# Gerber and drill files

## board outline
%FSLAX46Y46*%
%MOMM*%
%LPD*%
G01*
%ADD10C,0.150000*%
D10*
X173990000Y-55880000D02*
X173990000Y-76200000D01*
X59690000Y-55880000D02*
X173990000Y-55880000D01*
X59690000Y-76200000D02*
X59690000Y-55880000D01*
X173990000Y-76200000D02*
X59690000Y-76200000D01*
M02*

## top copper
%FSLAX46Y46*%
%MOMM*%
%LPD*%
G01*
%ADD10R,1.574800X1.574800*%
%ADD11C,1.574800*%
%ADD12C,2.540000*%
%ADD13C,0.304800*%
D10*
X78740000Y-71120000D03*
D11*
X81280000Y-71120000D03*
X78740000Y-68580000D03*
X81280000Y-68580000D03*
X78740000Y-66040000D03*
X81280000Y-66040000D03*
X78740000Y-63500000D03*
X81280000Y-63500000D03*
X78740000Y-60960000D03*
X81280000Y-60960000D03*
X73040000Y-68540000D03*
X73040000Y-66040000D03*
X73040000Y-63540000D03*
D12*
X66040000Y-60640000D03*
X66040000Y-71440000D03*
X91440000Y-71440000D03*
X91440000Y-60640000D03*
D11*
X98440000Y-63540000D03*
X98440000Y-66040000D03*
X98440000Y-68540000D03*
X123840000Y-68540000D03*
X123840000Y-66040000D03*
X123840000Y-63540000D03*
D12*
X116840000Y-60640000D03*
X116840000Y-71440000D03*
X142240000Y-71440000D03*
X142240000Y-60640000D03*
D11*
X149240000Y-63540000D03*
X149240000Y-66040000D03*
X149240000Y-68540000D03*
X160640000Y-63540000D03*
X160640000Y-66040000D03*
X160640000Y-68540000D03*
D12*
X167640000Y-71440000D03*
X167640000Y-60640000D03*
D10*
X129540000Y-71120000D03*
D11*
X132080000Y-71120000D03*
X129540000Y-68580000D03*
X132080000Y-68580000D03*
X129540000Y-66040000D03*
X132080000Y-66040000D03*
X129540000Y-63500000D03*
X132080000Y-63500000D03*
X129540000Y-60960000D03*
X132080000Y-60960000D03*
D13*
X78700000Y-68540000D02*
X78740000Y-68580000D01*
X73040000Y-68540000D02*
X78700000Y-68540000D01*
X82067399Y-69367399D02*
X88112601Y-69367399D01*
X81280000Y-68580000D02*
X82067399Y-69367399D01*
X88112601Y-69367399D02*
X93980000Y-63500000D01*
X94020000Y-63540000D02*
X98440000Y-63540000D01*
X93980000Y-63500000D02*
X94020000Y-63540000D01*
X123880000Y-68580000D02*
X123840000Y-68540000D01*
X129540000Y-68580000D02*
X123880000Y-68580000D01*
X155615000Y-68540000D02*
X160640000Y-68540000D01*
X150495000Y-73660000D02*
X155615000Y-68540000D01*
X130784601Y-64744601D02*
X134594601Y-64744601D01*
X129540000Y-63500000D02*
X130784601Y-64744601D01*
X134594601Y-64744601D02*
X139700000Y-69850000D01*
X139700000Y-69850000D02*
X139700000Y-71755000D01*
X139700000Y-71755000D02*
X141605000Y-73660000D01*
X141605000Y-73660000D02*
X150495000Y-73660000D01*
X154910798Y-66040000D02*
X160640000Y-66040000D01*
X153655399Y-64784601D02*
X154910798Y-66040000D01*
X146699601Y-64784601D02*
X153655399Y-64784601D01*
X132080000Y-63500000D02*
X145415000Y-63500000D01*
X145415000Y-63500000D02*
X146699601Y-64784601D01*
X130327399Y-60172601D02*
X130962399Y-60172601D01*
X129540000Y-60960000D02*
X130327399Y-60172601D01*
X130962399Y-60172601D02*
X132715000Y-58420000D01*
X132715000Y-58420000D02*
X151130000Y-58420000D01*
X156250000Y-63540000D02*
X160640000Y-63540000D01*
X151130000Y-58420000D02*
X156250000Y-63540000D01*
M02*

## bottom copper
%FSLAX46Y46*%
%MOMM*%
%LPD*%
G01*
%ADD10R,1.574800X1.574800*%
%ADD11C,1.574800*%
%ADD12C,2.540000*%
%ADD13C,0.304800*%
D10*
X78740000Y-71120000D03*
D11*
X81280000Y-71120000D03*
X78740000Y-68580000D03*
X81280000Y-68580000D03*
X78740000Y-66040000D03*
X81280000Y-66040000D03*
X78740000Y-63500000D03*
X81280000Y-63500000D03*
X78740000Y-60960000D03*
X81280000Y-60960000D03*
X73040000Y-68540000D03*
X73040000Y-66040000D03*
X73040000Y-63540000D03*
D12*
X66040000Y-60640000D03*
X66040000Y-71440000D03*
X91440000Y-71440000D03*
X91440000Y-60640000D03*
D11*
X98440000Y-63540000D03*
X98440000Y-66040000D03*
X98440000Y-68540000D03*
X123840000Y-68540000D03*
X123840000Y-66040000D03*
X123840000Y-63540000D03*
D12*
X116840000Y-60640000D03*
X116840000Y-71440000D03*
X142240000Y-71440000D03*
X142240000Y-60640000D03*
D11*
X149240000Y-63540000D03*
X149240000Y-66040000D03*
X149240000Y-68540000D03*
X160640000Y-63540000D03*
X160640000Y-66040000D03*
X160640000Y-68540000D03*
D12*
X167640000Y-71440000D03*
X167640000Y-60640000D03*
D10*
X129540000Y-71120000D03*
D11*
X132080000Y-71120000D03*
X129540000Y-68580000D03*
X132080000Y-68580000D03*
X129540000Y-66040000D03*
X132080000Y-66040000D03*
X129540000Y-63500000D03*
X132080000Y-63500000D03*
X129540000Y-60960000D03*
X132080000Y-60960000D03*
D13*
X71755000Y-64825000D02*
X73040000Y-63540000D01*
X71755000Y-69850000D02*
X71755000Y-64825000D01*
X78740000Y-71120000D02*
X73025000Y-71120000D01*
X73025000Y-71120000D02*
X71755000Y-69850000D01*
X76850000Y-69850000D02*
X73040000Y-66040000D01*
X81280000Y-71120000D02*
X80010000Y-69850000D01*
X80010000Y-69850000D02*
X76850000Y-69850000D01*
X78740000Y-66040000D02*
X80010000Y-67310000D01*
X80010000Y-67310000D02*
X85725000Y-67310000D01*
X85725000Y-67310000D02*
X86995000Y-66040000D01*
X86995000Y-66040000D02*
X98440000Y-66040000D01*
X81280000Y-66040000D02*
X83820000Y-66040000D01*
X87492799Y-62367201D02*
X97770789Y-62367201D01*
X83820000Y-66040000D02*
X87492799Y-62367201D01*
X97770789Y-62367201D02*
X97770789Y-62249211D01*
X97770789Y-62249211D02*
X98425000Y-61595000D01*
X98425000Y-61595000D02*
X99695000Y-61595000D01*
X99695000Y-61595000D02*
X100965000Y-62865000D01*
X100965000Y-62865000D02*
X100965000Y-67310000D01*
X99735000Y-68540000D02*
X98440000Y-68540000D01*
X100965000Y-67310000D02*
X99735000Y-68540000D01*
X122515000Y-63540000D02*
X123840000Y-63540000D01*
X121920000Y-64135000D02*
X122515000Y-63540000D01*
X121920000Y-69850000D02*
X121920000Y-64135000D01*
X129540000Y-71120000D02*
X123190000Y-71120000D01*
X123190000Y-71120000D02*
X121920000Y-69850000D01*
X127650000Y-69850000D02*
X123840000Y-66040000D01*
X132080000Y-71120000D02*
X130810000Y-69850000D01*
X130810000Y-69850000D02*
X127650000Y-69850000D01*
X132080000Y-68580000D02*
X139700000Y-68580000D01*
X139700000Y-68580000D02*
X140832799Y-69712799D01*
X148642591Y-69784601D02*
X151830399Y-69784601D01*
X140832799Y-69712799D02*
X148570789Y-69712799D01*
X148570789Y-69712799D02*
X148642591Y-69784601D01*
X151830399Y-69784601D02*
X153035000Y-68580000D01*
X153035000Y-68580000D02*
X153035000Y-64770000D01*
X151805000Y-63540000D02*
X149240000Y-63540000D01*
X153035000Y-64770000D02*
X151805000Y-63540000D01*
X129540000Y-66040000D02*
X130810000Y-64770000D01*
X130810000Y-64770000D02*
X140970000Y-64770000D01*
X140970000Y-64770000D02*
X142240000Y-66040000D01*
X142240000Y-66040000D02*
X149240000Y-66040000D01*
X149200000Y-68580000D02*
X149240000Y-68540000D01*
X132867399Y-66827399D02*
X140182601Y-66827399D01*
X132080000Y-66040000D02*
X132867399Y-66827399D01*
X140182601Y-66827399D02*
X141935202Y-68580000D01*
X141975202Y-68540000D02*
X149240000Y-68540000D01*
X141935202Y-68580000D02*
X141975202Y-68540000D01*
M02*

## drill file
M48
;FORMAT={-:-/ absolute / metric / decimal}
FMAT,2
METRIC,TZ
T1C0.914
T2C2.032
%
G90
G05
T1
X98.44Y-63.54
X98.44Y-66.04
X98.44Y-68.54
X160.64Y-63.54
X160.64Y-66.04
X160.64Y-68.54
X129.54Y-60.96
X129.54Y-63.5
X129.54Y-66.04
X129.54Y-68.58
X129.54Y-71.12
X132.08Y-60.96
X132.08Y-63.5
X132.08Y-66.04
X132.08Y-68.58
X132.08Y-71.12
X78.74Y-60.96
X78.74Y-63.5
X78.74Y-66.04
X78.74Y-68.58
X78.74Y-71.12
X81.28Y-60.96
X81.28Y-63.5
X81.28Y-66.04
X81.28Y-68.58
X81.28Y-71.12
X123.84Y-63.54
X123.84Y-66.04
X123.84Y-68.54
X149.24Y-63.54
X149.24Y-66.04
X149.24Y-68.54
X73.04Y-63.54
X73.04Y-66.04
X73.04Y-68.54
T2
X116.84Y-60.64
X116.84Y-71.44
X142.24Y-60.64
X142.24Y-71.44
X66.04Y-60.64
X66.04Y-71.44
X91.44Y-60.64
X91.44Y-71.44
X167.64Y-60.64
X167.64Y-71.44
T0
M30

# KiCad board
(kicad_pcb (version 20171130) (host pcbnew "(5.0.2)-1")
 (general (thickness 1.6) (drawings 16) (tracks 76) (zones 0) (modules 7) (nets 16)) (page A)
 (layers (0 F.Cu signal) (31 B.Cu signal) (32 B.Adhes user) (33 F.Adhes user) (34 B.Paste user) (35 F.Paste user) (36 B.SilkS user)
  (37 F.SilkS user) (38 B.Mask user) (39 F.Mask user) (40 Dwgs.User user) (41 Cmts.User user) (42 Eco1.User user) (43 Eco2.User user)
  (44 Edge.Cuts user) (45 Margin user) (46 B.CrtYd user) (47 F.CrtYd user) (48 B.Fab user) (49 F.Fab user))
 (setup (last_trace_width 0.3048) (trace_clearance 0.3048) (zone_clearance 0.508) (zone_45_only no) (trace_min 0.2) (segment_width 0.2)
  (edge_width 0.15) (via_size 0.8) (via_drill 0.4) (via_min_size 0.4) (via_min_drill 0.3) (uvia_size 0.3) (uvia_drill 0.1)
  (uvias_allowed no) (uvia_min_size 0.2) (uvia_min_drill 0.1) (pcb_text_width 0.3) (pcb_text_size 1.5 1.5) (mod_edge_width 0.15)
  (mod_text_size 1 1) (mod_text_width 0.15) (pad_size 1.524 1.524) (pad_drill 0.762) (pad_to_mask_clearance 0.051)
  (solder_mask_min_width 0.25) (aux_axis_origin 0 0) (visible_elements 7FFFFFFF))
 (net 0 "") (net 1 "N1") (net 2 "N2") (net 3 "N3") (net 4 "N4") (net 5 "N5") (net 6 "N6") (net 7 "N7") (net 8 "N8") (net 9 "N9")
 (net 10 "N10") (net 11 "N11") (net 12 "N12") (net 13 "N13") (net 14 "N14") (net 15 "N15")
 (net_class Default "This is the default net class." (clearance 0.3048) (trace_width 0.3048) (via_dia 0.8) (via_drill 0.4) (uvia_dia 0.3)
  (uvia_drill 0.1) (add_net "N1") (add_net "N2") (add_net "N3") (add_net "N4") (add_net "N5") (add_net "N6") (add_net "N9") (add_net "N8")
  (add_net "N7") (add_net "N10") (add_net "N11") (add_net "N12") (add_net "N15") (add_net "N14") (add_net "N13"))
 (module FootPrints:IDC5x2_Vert (layer B.Cu) (at 80.01 66.04 270)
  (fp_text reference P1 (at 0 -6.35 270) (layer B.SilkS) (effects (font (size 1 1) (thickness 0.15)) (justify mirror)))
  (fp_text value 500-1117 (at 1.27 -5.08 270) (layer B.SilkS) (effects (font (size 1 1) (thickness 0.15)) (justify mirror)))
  (pad 1 thru_hole rect (at 5.08 1.27 270) (size 1.5748 1.5748) (drill 0.9144) (layers *.Cu *.Mask B.SilkS) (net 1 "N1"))
  (pad 2 thru_hole circle (at 5.08 -1.27 270) (size 1.5748 1.5748) (drill 0.9144) (layers *.Cu *.Mask B.SilkS) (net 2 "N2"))
  (pad 3 thru_hole circle (at 2.54 1.27 270) (size 1.5748 1.5748) (drill 0.9144) (layers *.Cu *.Mask B.SilkS) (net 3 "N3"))
  (pad 4 thru_hole circle (at 2.54 -1.27 270) (size 1.5748 1.5748) (drill 0.9144) (layers *.Cu *.Mask B.SilkS) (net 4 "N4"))
  (pad 5 thru_hole circle (at 0 1.27 270) (size 1.5748 1.5748) (drill 0.9144) (layers *.Cu *.Mask B.SilkS) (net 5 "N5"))
  (pad 6 thru_hole circle (at 0 -1.27 270) (size 1.5748 1.5748) (drill 0.9144) (layers *.Cu *.Mask B.SilkS) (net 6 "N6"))
  (pad 7 thru_hole circle (at -2.54 1.27 270) (size 1.5748 1.5748) (drill 0.9144) (layers *.Cu *.Mask B.SilkS))
  (pad 8 thru_hole circle (at -2.54 -1.27 270) (size 1.5748 1.5748) (drill 0.9144) (layers *.Cu *.Mask B.SilkS))
  (pad 9 thru_hole circle (at -5.08 1.27 270) (size 1.5748 1.5748) (drill 0.9144) (layers *.Cu *.Mask B.SilkS))
  (pad 10 thru_hole circle (at -5.08 -1.27 270) (size 1.5748 1.5748) (drill 0.9144) (layers *.Cu *.Mask B.SilkS)))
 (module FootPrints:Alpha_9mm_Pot (layer F.Cu) (at 66.04 66.04 90)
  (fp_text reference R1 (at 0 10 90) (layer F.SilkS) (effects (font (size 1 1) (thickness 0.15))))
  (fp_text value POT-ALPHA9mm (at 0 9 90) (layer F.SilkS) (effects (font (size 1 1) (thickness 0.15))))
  (pad 1 thru_hole circle (at -2.5 7 90) (size 1.5748 1.5748) (drill 0.9144) (layers *.Cu *.Mask) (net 3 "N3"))
  (pad 2 thru_hole circle (at 0 7 90) (size 1.5748 1.5748) (drill 0.9144) (layers *.Cu *.Mask) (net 2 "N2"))
  (pad 3 thru_hole circle (at 2.5 7 90) (size 1.5748 1.5748) (drill 0.9144) (layers *.Cu *.Mask) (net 1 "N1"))
  (pad 4 thru_hole circle (at 5.4 0 90) (size 2.54 2.54) (drill 2.032) (layers *.Cu *.Mask))
  (pad 5 thru_hole circle (at -5.4 0 90) (size 2.54 2.54) (drill 2.032) (layers *.Cu *.Mask)))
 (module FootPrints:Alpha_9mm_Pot (layer F.Cu) (at 91.44 66.04 90)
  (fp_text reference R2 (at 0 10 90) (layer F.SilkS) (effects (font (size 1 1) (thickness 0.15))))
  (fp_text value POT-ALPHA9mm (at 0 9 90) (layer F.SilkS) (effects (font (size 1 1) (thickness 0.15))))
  (pad 5 thru_hole circle (at -5.4 0 90) (size 2.54 2.54) (drill 2.032) (layers *.Cu *.Mask))
  (pad 4 thru_hole circle (at 5.4 0 90) (size 2.54 2.54) (drill 2.032) (layers *.Cu *.Mask))
  (pad 3 thru_hole circle (at 2.5 7 90) (size 1.5748 1.5748) (drill 0.9144) (layers *.Cu *.Mask) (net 4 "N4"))
  (pad 2 thru_hole circle (at 0 7 90) (size 1.5748 1.5748) (drill 0.9144) (layers *.Cu *.Mask) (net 5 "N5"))
  (pad 1 thru_hole circle (at -2.5 7 90) (size 1.5748 1.5748) (drill 0.9144) (layers *.Cu *.Mask) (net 6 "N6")))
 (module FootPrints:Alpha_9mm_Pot (layer F.Cu) (at 116.84 66.04 90)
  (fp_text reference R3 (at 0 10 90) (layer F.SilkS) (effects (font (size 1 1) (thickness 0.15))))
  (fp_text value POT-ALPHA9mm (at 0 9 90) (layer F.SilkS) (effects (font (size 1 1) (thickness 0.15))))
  (pad 1 thru_hole circle (at -2.5 7 90) (size 1.5748 1.5748) (drill 0.9144) (layers *.Cu *.Mask) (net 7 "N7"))
  (pad 2 thru_hole circle (at 0 7 90) (size 1.5748 1.5748) (drill 0.9144) (layers *.Cu *.Mask) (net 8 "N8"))
  (pad 3 thru_hole circle (at 2.5 7 90) (size 1.5748 1.5748) (drill 0.9144) (layers *.Cu *.Mask) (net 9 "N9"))
  (pad 4 thru_hole circle (at 5.4 0 90) (size 2.54 2.54) (drill 2.032) (layers *.Cu *.Mask))
  (pad 5 thru_hole circle (at -5.4 0 90) (size 2.54 2.54) (drill 2.032) (layers *.Cu *.Mask)))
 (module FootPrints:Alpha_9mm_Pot (layer F.Cu) (at 142.24 66.04 90)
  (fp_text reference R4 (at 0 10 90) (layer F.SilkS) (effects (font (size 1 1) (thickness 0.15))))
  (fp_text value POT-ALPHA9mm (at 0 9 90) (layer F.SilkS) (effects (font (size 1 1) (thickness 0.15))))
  (pad 5 thru_hole circle (at -5.4 0 90) (size 2.54 2.54) (drill 2.032) (layers *.Cu *.Mask))
  (pad 4 thru_hole circle (at 5.4 0 90) (size 2.54 2.54) (drill 2.032) (layers *.Cu *.Mask))
  (pad 3 thru_hole circle (at 2.5 7 90) (size 1.5748 1.5748) (drill 0.9144) (layers *.Cu *.Mask) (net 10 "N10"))
  (pad 2 thru_hole circle (at 0 7 90) (size 1.5748 1.5748) (drill 0.9144) (layers *.Cu *.Mask) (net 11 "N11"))
  (pad 1 thru_hole circle (at -2.5 7 90) (size 1.5748 1.5748) (drill 0.9144) (layers *.Cu *.Mask) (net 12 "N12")))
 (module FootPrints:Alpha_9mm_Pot (layer F.Cu) (at 167.64 66.04 270)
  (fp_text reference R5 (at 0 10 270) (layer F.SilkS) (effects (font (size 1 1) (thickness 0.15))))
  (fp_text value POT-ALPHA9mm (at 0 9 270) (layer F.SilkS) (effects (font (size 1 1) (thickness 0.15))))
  (pad 1 thru_hole circle (at -2.5 7 270) (size 1.5748 1.5748) (drill 0.9144) (layers *.Cu *.Mask) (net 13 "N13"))
  (pad 2 thru_hole circle (at 0 7 270) (size 1.5748 1.5748) (drill 0.9144) (layers *.Cu *.Mask) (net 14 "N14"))
  (pad 3 thru_hole circle (at 2.5 7 270) (size 1.5748 1.5748) (drill 0.9144) (layers *.Cu *.Mask) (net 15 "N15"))
  (pad 4 thru_hole circle (at 5.4 0 270) (size 2.54 2.54) (drill 2.032) (layers *.Cu *.Mask))
  (pad 5 thru_hole circle (at -5.4 0 270) (size 2.54 2.54) (drill 2.032) (layers *.Cu *.Mask)))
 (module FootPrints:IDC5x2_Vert (layer B.Cu) (at 130.81 66.04 270)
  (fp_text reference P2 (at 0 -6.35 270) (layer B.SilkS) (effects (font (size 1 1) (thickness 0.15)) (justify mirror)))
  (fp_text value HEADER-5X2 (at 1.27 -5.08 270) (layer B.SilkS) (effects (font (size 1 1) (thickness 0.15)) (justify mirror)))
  (pad 1 thru_hole rect (at 5.08 1.27 270) (size 1.5748 1.5748) (drill 0.9144) (layers *.Cu *.Mask B.SilkS) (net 9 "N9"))
  (pad 2 thru_hole circle (at 5.08 -1.27 270) (size 1.5748 1.5748) (drill 0.9144) (layers *.Cu *.Mask B.SilkS) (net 8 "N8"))
  (pad 3 thru_hole circle (at 2.54 1.27 270) (size 1.5748 1.5748) (drill 0.9144) (layers *.Cu *.Mask B.SilkS) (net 7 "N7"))
  (pad 4 thru_hole circle (at 2.54 -1.27 270) (size 1.5748 1.5748) (drill 0.9144) (layers *.Cu *.Mask B.SilkS) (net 10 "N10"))
  (pad 5 thru_hole circle (at 0 1.27 270) (size 1.5748 1.5748) (drill 0.9144) (layers *.Cu *.Mask B.SilkS) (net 11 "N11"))
  (pad 6 thru_hole circle (at 0 -1.27 270) (size 1.5748 1.5748) (drill 0.9144) (layers *.Cu *.Mask B.SilkS) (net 12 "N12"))
  (pad 7 thru_hole circle (at -2.54 1.27 270) (size 1.5748 1.5748) (drill 0.9144) (layers *.Cu *.Mask B.SilkS) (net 15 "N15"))
  (pad 8 thru_hole circle (at -2.54 -1.27 270) (size 1.5748 1.5748) (drill 0.9144) (layers *.Cu *.Mask B.SilkS) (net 14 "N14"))
  (pad 9 thru_hole circle (at -5.08 1.27 270) (size 1.5748 1.5748) (drill 0.9144) (layers *.Cu *.Mask B.SilkS) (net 13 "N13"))
  (pad 10 thru_hole circle (at -5.08 -1.27 270) (size 1.5748 1.5748) (drill 0.9144) (layers *.Cu *.Mask B.SilkS)))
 (gr_line (start 173.99 55.88) (end 173.99 76.2) (layer Edge.Cuts) (width 0.15))
 (gr_line (start 59.69 55.88) (end 173.99 55.88) (layer Edge.Cuts) (width 0.15))
 (gr_line (start 59.69 76.2) (end 59.69 55.88) (layer Edge.Cuts) (width 0.15))
 (gr_line (start 173.99 76.2) (end 59.69 76.2) (layer Edge.Cuts) (width 0.15))
 (segment (start 71.755 64.825) (end 73.04 63.54) (width 0.3048) (layer B.Cu) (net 1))
 (segment (start 71.755 69.85) (end 71.755 64.825) (width 0.3048) (layer B.Cu) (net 1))
 (segment (start 78.74 71.12) (end 73.025 71.12) (width 0.3048) (layer B.Cu) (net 1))
 (segment (start 73.025 71.12) (end 71.755 69.85) (width 0.3048) (layer B.Cu) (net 1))
 (segment (start 76.85 69.85) (end 73.04 66.04) (width 0.3048) (layer B.Cu) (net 2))
 (segment (start 81.28 71.12) (end 80.01 69.85) (width 0.3048) (layer B.Cu) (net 2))
 (segment (start 80.01 69.85) (end 76.85 69.85) (width 0.3048) (layer B.Cu) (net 2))
 (segment (start 78.7 68.54) (end 78.74 68.58) (width 0.3048) (layer F.Cu) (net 3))
 (segment (start 73.04 68.54) (end 78.7 68.54) (width 0.3048) (layer F.Cu) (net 3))
 (segment (start 82.067399 69.367399) (end 88.112601 69.367399) (width 0.3048) (layer F.Cu) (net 4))
 (segment (start 81.28 68.58) (end 82.067399 69.367399) (width 0.3048) (layer F.Cu) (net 4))
 (segment (start 88.112601 69.367399) (end 93.98 63.5) (width 0.3048) (layer F.Cu) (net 4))
 (segment (start 94.02 63.54) (end 98.44 63.54) (width 0.3048) (layer F.Cu) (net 4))
 (segment (start 93.98 63.5) (end 94.02 63.54) (width 0.3048) (layer F.Cu) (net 4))
 (segment (start 78.74 66.04) (end 80.01 67.31) (width 0.3048) (layer B.Cu) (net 5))
 (segment (start 80.01 67.31) (end 85.725 67.31) (width 0.3048) (layer B.Cu) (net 5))
 (segment (start 85.725 67.31) (end 86.995 66.04) (width 0.3048) (layer B.Cu) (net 5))
 (segment (start 86.995 66.04) (end 98.44 66.04) (width 0.3048) (layer B.Cu) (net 5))
 (segment (start 81.28 66.04) (end 83.82 66.04) (width 0.3048) (layer B.Cu) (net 6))
 (segment (start 87.492799 62.367201) (end 97.770789 62.367201) (width 0.3048) (layer B.Cu) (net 6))
 (segment (start 83.82 66.04) (end 87.492799 62.367201) (width 0.3048) (layer B.Cu) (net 6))
 (segment (start 97.770789 62.367201) (end 97.770789 62.249211) (width 0.3048) (layer B.Cu) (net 6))
 (segment (start 97.770789 62.249211) (end 98.425 61.595) (width 0.3048) (layer B.Cu) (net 6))
 (segment (start 98.425 61.595) (end 99.695 61.595) (width 0.3048) (layer B.Cu) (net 6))
 (segment (start 99.695 61.595) (end 100.965 62.865) (width 0.3048) (layer B.Cu) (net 6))
 (segment (start 100.965 62.865) (end 100.965 67.31) (width 0.3048) (layer B.Cu) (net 6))
 (segment (start 99.735 68.54) (end 98.44 68.54) (width 0.3048) (layer B.Cu) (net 6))
 (segment (start 100.965 67.31) (end 99.735 68.54) (width 0.3048) (layer B.Cu) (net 6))
 (segment (start 122.515 63.54) (end 123.84 63.54) (width 0.3048) (layer B.Cu) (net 9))
 (segment (start 121.92 64.135) (end 122.515 63.54) (width 0.3048) (layer B.Cu) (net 9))
 (segment (start 121.92 69.85) (end 121.92 64.135) (width 0.3048) (layer B.Cu) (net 9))
 (segment (start 129.54 71.12) (end 123.19 71.12) (width 0.3048) (layer B.Cu) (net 9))
 (segment (start 123.19 71.12) (end 121.92 69.85) (width 0.3048) (layer B.Cu) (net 9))
 (segment (start 127.65 69.85) (end 123.84 66.04) (width 0.3048) (layer B.Cu) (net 8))
 (segment (start 132.08 71.12) (end 130.81 69.85) (width 0.3048) (layer B.Cu) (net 8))
 (segment (start 130.81 69.85) (end 127.65 69.85) (width 0.3048) (layer B.Cu) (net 8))
 (segment (start 123.88 68.58) (end 123.84 68.54) (width 0.3048) (layer F.Cu) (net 7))
 (segment (start 129.54 68.58) (end 123.88 68.58) (width 0.3048) (layer F.Cu) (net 7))
 (segment (start 132.08 68.58) (end 139.7 68.58) (width 0.3048) (layer B.Cu) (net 10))
 (segment (start 139.7 68.58) (end 140.832799 69.712799) (width 0.3048) (layer B.Cu) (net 10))
 (segment (start 148.642591 69.784601) (end 151.830399 69.784601) (width 0.3048) (layer B.Cu) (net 10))
 (segment (start 140.832799 69.712799) (end 148.570789 69.712799) (width 0.3048) (layer B.Cu) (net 10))
 (segment (start 148.570789 69.712799) (end 148.642591 69.784601) (width 0.3048) (layer B.Cu) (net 10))
 (segment (start 151.830399 69.784601) (end 153.035 68.58) (width 0.3048) (layer B.Cu) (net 10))
 (segment (start 153.035 68.58) (end 153.035 64.77) (width 0.3048) (layer B.Cu) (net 10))
 (segment (start 151.805 63.54) (end 149.24 63.54) (width 0.3048) (layer B.Cu) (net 10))
 (segment (start 153.035 64.77) (end 151.805 63.54) (width 0.3048) (layer B.Cu) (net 10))
 (segment (start 129.54 66.04) (end 130.81 64.77) (width 0.3048) (layer B.Cu) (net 11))
 (segment (start 130.81 64.77) (end 140.97 64.77) (width 0.3048) (layer B.Cu) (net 11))
 (segment (start 140.97 64.77) (end 142.24 66.04) (width 0.3048) (layer B.Cu) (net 11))
 (segment (start 142.24 66.04) (end 149.24 66.04) (width 0.3048) (layer B.Cu) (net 11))
 (segment (start 149.2 68.58) (end 149.24 68.54) (width 0.3048) (layer B.Cu) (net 12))
 (segment (start 132.867399 66.827399) (end 140.182601 66.827399) (width 0.3048) (layer B.Cu) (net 12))
 (segment (start 132.08 66.04) (end 132.867399 66.827399) (width 0.3048) (layer B.Cu) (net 12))
 (segment (start 140.182601 66.827399) (end 141.935202 68.58) (width 0.3048) (layer B.Cu) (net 12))
 (segment (start 141.975202 68.54) (end 149.24 68.54) (width 0.3048) (layer B.Cu) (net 12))
 (segment (start 141.935202 68.58) (end 141.975202 68.54) (width 0.3048) (layer B.Cu) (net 12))
 (segment (start 155.615 68.54) (end 160.64 68.54) (width 0.3048) (layer F.Cu) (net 15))
 (segment (start 150.495 73.66) (end 155.615 68.54) (width 0.3048) (layer F.Cu) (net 15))
 (segment (start 130.784601 64.744601) (end 134.594601 64.744601) (width 0.3048) (layer F.Cu) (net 15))
 (segment (start 129.54 63.5) (end 130.784601 64.744601) (width 0.3048) (layer F.Cu) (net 15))
 (segment (start 134.594601 64.744601) (end 139.7 69.85) (width 0.3048) (layer F.Cu) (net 15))
 (segment (start 139.7 69.85) (end 139.7 71.755) (width 0.3048) (layer F.Cu) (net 15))
 (segment (start 139.7 71.755) (end 141.605 73.66) (width 0.3048) (layer F.Cu) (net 15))
 (segment (start 141.605 73.66) (end 150.495 73.66) (width 0.3048) (layer F.Cu) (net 15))
 (segment (start 154.910798 66.04) (end 160.64 66.04) (width 0.3048) (layer F.Cu) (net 14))
 (segment (start 153.655399 64.784601) (end 154.910798 66.04) (width 0.3048) (layer F.Cu) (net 14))
 (segment (start 146.699601 64.784601) (end 153.655399 64.784601) (width 0.3048) (layer F.Cu) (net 14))
 (segment (start 132.08 63.5) (end 145.415 63.5) (width 0.3048) (layer F.Cu) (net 14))
 (segment (start 145.415 63.5) (end 146.699601 64.784601) (width 0.3048) (layer F.Cu) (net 14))
 (segment (start 130.327399 60.172601) (end 130.962399 60.172601) (width 0.3048) (layer F.Cu) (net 13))
 (segment (start 129.54 60.96) (end 130.327399 60.172601) (width 0.3048) (layer F.Cu) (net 13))
 (segment (start 130.962399 60.172601) (end 132.715 58.42) (width 0.3048) (layer F.Cu) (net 13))
 (segment (start 132.715 58.42) (end 151.13 58.42) (width 0.3048) (layer F.Cu) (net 13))
 (segment (start 156.25 63.54) (end 160.64 63.54) (width 0.3048) (layer F.Cu) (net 13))
 (segment (start 151.13 58.42) (end 156.25 63.54) (width 0.3048) (layer F.Cu) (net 13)))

